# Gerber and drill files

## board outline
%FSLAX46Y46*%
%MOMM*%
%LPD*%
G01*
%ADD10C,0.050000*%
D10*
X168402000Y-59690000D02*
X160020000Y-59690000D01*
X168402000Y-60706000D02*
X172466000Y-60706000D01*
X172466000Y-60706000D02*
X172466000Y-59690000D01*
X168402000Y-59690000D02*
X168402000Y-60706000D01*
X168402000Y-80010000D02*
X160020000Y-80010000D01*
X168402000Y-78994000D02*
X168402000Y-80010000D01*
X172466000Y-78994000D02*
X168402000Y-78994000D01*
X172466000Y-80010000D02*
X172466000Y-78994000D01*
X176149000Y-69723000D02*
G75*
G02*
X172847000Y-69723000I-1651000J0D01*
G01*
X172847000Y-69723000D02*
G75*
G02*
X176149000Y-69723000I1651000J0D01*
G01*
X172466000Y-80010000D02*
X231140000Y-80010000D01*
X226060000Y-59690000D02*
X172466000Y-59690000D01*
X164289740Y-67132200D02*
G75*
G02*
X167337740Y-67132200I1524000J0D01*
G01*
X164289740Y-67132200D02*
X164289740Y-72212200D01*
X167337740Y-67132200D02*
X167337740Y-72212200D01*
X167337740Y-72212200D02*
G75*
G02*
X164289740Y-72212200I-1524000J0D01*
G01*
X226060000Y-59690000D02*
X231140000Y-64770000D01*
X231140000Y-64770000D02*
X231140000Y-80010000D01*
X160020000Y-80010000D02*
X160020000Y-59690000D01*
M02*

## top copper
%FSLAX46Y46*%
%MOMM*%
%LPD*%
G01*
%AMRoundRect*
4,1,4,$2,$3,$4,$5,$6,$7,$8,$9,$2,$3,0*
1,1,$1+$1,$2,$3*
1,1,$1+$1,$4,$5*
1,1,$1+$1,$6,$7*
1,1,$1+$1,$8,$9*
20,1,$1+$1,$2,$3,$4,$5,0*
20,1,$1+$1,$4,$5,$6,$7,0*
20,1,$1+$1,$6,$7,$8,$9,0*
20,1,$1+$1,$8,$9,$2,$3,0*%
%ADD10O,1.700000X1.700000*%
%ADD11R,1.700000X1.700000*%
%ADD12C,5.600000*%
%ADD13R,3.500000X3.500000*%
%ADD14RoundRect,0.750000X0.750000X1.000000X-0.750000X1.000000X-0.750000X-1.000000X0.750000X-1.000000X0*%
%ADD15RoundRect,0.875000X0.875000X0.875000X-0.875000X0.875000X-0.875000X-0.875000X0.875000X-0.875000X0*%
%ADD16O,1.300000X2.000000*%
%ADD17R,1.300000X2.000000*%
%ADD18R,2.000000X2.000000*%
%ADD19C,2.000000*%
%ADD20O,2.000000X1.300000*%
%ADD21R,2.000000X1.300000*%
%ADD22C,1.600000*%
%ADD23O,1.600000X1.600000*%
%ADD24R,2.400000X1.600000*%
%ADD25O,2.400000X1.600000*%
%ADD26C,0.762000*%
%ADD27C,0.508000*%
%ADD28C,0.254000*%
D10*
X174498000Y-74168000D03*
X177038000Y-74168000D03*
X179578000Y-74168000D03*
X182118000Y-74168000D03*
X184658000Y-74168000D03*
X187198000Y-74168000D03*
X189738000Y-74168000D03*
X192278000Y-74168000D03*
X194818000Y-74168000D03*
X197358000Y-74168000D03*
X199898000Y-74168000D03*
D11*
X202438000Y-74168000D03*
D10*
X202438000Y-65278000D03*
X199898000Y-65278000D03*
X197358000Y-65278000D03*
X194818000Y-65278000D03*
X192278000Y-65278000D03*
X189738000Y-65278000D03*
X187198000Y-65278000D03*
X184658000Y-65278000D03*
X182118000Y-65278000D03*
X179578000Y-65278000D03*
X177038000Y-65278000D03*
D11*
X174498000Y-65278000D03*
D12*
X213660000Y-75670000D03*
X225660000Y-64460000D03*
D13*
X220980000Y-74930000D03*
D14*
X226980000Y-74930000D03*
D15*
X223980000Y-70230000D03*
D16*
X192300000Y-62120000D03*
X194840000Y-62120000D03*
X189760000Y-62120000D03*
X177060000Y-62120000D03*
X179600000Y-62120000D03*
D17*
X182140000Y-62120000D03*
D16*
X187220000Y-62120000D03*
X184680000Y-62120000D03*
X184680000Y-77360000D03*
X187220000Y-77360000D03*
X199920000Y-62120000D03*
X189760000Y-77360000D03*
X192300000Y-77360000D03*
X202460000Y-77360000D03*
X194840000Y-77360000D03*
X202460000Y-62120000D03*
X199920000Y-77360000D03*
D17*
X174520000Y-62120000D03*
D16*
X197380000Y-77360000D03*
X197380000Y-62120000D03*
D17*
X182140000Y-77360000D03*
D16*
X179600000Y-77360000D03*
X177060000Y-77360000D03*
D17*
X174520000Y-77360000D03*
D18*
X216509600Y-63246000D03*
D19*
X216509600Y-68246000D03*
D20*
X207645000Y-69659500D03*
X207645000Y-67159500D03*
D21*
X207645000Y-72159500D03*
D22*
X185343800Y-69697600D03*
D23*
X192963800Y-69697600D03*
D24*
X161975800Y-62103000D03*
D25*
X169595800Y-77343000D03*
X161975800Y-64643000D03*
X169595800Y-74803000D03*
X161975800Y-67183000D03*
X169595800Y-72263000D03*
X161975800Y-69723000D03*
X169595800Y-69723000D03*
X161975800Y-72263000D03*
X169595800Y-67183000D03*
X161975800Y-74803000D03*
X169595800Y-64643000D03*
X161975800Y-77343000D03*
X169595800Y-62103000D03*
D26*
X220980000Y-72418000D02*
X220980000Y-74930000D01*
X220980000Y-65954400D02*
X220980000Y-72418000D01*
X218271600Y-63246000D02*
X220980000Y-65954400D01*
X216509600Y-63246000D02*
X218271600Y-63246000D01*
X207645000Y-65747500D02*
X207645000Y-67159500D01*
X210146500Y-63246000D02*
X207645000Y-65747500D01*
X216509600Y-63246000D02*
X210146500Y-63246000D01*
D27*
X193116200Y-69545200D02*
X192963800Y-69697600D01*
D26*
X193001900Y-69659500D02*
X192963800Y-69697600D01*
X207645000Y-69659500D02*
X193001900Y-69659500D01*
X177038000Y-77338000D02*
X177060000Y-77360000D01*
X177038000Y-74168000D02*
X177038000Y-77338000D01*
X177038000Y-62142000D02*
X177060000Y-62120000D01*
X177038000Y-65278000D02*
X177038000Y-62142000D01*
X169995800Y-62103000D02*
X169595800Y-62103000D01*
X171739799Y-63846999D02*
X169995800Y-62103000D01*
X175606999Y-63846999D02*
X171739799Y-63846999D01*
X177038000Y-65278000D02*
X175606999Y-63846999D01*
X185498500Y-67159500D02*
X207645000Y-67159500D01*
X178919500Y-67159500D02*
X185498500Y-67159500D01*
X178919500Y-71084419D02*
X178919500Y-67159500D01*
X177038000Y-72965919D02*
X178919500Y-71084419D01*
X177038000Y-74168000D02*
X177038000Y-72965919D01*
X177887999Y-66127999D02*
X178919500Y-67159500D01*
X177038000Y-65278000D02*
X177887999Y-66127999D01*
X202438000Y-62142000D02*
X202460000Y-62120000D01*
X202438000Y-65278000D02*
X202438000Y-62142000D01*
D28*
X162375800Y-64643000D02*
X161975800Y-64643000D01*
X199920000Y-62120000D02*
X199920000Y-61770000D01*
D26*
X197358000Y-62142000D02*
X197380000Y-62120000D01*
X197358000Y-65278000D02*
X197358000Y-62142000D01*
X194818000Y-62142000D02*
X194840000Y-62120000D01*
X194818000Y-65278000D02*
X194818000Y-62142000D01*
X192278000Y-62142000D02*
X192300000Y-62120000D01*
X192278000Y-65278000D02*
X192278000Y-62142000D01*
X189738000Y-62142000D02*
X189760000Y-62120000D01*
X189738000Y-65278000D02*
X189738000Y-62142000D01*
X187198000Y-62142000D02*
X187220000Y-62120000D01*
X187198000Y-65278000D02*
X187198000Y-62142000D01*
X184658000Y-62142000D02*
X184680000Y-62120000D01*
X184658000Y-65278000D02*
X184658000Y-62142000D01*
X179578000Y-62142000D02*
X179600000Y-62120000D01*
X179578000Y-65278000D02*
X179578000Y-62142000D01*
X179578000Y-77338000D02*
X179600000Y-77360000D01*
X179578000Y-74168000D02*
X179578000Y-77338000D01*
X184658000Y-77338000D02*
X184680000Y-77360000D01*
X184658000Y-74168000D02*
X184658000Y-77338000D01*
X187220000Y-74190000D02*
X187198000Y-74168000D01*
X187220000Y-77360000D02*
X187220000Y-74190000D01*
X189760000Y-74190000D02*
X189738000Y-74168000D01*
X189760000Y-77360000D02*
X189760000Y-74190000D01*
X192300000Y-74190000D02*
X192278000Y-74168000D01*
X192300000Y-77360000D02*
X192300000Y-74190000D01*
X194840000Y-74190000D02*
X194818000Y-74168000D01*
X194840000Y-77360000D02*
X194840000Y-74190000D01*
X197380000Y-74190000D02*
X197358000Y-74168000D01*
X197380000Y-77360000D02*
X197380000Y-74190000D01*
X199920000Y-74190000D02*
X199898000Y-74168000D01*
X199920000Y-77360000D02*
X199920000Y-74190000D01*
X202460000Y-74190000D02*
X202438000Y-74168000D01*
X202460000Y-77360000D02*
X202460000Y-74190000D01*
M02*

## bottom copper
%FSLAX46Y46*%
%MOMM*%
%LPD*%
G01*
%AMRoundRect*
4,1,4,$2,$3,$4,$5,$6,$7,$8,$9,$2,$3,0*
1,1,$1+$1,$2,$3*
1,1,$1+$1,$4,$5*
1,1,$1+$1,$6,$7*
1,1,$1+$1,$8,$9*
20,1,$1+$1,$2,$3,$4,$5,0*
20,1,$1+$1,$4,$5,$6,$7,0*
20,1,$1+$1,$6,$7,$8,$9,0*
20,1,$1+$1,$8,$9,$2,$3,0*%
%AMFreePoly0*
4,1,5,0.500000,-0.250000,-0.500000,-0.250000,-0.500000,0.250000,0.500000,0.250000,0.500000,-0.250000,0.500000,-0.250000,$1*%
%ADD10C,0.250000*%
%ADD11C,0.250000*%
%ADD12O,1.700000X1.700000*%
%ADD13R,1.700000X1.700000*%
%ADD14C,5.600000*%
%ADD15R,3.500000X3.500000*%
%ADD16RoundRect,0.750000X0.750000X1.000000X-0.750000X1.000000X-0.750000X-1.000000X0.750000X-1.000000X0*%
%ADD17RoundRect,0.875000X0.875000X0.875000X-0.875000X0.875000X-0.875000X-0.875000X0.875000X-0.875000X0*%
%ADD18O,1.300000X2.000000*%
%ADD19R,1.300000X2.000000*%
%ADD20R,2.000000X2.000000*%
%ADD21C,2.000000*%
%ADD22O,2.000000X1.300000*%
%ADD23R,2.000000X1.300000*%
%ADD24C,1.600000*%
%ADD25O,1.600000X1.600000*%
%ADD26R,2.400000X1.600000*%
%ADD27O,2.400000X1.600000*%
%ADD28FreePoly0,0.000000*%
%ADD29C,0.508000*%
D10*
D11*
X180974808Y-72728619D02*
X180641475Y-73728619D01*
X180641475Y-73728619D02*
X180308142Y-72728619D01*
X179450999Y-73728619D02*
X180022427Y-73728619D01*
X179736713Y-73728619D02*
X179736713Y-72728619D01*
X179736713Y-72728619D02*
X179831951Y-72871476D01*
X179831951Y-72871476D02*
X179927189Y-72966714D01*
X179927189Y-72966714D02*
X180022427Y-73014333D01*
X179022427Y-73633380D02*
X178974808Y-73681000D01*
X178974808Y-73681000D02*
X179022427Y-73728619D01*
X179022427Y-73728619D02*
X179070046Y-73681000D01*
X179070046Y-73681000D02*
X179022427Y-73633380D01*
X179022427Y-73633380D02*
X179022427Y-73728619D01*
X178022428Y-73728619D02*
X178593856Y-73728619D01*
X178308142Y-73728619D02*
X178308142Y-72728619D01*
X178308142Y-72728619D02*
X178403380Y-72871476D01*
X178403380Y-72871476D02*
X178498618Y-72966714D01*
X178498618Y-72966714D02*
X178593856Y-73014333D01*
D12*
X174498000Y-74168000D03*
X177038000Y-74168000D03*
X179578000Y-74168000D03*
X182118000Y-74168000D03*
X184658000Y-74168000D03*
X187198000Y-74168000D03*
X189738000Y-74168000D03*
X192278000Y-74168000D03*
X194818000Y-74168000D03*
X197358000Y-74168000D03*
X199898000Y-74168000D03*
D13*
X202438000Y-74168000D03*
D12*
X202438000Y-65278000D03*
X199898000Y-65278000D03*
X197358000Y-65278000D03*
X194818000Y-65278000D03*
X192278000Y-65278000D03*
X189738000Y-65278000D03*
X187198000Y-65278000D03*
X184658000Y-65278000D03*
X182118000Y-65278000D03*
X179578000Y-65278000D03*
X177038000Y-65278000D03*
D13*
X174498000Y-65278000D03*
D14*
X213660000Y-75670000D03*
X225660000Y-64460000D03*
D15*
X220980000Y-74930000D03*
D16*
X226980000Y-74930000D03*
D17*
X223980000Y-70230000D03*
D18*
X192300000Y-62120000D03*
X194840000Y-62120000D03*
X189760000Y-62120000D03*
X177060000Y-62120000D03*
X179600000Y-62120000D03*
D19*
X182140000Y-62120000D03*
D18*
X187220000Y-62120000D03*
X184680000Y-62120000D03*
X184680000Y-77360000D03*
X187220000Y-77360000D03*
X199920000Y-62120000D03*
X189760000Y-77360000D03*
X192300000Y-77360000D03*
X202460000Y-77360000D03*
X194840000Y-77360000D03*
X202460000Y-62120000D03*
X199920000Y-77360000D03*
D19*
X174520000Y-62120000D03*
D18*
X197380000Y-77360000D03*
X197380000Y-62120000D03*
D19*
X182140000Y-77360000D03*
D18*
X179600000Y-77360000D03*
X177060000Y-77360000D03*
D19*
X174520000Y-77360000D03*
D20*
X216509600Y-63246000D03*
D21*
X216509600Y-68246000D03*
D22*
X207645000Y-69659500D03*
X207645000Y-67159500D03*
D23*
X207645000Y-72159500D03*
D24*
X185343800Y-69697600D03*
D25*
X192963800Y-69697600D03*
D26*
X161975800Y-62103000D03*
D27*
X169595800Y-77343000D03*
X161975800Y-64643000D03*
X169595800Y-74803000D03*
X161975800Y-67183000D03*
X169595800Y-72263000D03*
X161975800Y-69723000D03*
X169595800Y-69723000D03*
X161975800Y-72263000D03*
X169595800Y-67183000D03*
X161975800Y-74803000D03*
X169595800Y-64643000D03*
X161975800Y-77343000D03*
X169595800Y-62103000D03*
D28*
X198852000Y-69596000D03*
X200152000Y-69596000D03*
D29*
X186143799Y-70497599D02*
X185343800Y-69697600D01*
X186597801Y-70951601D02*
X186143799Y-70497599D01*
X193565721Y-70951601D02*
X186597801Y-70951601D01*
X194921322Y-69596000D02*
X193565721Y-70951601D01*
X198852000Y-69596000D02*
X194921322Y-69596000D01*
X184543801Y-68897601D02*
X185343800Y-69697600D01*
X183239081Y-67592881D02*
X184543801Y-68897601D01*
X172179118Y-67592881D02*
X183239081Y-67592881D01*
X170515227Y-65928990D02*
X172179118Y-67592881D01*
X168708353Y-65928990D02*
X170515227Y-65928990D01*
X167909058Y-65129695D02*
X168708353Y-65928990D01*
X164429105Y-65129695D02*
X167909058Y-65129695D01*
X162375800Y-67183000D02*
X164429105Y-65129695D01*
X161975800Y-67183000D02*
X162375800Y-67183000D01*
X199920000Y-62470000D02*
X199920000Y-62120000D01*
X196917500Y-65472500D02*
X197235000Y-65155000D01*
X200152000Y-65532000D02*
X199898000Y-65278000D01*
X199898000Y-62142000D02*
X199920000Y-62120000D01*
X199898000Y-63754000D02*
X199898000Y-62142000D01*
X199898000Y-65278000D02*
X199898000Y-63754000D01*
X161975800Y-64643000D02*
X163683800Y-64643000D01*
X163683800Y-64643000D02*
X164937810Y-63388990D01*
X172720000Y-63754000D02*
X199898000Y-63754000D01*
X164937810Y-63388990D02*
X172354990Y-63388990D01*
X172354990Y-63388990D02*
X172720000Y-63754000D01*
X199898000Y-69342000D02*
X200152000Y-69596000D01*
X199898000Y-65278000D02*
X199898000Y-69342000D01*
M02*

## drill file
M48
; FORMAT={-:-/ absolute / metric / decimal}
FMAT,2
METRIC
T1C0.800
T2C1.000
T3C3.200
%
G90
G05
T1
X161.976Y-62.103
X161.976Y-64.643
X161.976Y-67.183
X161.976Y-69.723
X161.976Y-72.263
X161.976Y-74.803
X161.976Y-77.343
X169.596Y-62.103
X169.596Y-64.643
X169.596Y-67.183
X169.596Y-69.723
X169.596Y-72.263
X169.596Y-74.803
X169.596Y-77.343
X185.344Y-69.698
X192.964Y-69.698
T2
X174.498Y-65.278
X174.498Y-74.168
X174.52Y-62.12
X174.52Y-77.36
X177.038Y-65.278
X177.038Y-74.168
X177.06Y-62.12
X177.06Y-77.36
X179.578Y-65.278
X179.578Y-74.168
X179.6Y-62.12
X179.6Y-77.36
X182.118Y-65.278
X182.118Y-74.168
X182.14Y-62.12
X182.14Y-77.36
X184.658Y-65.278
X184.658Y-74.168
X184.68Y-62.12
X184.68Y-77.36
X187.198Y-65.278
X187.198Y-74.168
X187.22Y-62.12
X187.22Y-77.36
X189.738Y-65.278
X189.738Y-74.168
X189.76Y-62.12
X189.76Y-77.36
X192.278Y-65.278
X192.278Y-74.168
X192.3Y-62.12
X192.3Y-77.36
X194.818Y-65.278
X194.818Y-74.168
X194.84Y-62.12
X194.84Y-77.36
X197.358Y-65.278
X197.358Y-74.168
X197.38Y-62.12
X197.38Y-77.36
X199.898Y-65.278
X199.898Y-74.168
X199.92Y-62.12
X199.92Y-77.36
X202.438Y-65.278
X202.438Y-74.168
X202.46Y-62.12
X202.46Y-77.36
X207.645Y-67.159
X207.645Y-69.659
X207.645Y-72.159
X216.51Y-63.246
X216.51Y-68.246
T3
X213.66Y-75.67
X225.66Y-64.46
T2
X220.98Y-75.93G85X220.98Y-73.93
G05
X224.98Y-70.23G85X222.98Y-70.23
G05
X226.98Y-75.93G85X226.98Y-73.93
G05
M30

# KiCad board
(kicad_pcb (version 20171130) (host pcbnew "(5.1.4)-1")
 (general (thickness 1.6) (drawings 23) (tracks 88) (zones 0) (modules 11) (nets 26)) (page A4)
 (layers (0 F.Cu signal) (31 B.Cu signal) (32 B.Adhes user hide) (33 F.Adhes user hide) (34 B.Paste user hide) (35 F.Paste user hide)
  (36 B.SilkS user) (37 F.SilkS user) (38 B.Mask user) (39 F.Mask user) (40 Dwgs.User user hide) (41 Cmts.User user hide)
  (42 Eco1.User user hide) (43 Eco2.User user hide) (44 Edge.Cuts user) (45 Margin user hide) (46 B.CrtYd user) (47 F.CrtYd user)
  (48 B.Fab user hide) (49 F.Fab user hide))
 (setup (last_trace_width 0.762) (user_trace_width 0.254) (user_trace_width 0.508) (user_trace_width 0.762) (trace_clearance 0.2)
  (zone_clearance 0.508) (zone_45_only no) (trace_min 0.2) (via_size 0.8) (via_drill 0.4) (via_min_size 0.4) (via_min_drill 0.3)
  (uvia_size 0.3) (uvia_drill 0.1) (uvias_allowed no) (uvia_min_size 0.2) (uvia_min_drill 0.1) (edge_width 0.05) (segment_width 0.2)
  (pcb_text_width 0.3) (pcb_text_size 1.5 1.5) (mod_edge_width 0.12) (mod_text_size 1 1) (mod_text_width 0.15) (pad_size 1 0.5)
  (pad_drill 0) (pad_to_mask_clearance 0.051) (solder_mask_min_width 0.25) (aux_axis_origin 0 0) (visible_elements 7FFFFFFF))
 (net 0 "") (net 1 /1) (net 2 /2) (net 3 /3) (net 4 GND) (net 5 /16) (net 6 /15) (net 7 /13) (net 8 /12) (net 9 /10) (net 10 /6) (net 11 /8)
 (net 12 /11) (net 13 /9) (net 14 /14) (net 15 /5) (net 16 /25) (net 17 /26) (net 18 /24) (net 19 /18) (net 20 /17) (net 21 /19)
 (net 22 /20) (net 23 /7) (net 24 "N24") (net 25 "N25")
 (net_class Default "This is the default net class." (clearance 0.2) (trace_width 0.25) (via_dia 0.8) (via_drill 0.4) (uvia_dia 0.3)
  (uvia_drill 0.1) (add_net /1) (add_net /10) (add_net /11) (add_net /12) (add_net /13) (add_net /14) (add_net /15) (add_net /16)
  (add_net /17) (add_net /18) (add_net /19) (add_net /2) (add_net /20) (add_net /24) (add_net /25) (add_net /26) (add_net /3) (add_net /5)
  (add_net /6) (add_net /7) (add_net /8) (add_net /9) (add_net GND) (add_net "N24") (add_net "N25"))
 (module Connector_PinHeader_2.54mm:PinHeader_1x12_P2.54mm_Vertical (layer F.Cu) (at 202.438 74.168 270)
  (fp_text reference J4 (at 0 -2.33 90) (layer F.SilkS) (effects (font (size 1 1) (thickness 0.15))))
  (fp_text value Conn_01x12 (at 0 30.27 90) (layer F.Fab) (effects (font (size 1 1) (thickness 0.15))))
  (pad 12 thru_hole oval (at 0 27.94 270) (size 1.7 1.7) (drill 1) (layers *.Cu *.Mask) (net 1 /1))
  (pad 11 thru_hole oval (at 0 25.4 270) (size 1.7 1.7) (drill 1) (layers *.Cu *.Mask) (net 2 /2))
  (pad 10 thru_hole oval (at 0 22.86 270) (size 1.7 1.7) (drill 1) (layers *.Cu *.Mask) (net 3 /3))
  (pad 9 thru_hole oval (at 0 20.32 270) (size 1.7 1.7) (drill 1) (layers *.Cu *.Mask) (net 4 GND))
  (pad 8 thru_hole oval (at 0 17.78 270) (size 1.7 1.7) (drill 1) (layers *.Cu *.Mask) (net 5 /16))
  (pad 7 thru_hole oval (at 0 15.24 270) (size 1.7 1.7) (drill 1) (layers *.Cu *.Mask) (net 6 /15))
  (pad 6 thru_hole oval (at 0 12.7 270) (size 1.7 1.7) (drill 1) (layers *.Cu *.Mask) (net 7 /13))
  (pad 5 thru_hole oval (at 0 10.16 270) (size 1.7 1.7) (drill 1) (layers *.Cu *.Mask) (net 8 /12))
  (pad 4 thru_hole oval (at 0 7.62 270) (size 1.7 1.7) (drill 1) (layers *.Cu *.Mask) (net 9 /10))
  (pad 3 thru_hole oval (at 0 5.08 270) (size 1.7 1.7) (drill 1) (layers *.Cu *.Mask) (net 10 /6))
  (pad 2 thru_hole oval (at 0 2.54 270) (size 1.7 1.7) (drill 1) (layers *.Cu *.Mask) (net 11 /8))
  (pad 1 thru_hole rect (at 0 0 270) (size 1.7 1.7) (drill 1) (layers *.Cu *.Mask) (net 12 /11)))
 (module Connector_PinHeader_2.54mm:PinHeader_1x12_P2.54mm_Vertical (layer F.Cu) (at 174.498 65.278 90)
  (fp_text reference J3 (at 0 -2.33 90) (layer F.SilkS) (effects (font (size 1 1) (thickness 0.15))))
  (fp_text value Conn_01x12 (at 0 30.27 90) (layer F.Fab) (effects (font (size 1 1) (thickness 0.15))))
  (pad 12 thru_hole oval (at 0 27.94 90) (size 1.7 1.7) (drill 1) (layers *.Cu *.Mask) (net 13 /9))
  (pad 11 thru_hole oval (at 0 25.4 90) (size 1.7 1.7) (drill 1) (layers *.Cu *.Mask) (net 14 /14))
  (pad 10 thru_hole oval (at 0 22.86 90) (size 1.7 1.7) (drill 1) (layers *.Cu *.Mask) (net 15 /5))
  (pad 9 thru_hole oval (at 0 20.32 90) (size 1.7 1.7) (drill 1) (layers *.Cu *.Mask) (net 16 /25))
  (pad 8 thru_hole oval (at 0 17.78 90) (size 1.7 1.7) (drill 1) (layers *.Cu *.Mask) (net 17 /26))
  (pad 7 thru_hole oval (at 0 15.24 90) (size 1.7 1.7) (drill 1) (layers *.Cu *.Mask) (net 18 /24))
  (pad 6 thru_hole oval (at 0 12.7 90) (size 1.7 1.7) (drill 1) (layers *.Cu *.Mask) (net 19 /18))
  (pad 5 thru_hole oval (at 0 10.16 90) (size 1.7 1.7) (drill 1) (layers *.Cu *.Mask) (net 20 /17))
  (pad 4 thru_hole oval (at 0 7.62 90) (size 1.7 1.7) (drill 1) (layers *.Cu *.Mask) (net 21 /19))
  (pad 3 thru_hole oval (at 0 5.08 90) (size 1.7 1.7) (drill 1) (layers *.Cu *.Mask) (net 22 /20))
  (pad 2 thru_hole oval (at 0 2.54 90) (size 1.7 1.7) (drill 1) (layers *.Cu *.Mask) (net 2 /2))
  (pad 1 thru_hole rect (at 0 0 90) (size 1.7 1.7) (drill 1) (layers *.Cu *.Mask) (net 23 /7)))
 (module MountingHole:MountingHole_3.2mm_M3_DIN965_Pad (layer F.Cu) (at 213.66 75.67)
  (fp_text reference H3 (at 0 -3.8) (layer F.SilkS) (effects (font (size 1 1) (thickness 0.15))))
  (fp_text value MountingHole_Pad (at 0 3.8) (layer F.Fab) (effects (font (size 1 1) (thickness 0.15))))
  (pad 1 thru_hole circle (at 0 0) (size 5.6 5.6) (drill 3.2) (layers *.Cu *.Mask) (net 4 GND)))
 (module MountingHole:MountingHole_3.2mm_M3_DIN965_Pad (layer F.Cu) (at 225.66 64.46)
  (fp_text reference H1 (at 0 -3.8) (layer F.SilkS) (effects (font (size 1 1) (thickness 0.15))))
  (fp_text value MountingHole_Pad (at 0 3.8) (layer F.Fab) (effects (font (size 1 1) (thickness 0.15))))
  (pad 1 thru_hole circle (at 0 0) (size 5.6 5.6) (drill 3.2) (layers *.Cu *.Mask) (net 4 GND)))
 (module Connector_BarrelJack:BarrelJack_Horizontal (layer F.Cu) (at 220.98 74.93 180)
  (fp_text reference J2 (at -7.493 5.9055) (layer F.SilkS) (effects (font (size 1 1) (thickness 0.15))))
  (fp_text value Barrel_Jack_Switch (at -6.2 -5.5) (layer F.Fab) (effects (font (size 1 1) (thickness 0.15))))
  (pad 1 thru_hole rect (at 0 0 180) (size 3.5 3.5) (drill oval 1 3) (layers *.Cu *.Mask) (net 2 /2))
  (pad 2 thru_hole roundrect (at -6 0 180) (size 3 3.5) (drill oval 1 3) (layers *.Cu *.Mask) (roundrect_rratio 0.25) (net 1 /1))
  (pad 3 thru_hole roundrect (at -3 4.7 180) (size 3.5 3.5) (drill oval 3 1) (layers *.Cu *.Mask) (roundrect_rratio 0.25) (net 1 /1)))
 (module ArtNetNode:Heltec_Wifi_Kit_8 (layer F.Cu) (at 160.02 78.74)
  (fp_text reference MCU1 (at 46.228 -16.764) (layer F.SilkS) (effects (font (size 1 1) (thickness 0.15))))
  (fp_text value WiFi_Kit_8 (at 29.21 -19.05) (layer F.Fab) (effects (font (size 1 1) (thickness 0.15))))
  (pad 26 thru_hole oval (at 32.28 -16.62) (size 1.3 2) (drill 1) (layers *.Cu *.Mask) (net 17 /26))
  (pad 25 thru_hole oval (at 34.82 -16.62) (size 1.3 2) (drill 1) (layers *.Cu *.Mask) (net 16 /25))
  (pad 24 thru_hole oval (at 29.74 -16.62) (size 1.3 2) (drill 1) (layers *.Cu *.Mask) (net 18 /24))
  (pad 21 thru_hole oval (at 17.04 -16.62) (size 1.3 2) (drill 1) (layers *.Cu *.Mask) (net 2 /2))
  (pad 20 thru_hole oval (at 19.58 -16.62) (size 1.3 2) (drill 1) (layers *.Cu *.Mask) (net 22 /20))
  (pad 19 thru_hole rect (at 22.12 -16.62) (size 1.3 2) (drill 1) (layers *.Cu *.Mask) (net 21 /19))
  (pad 18 thru_hole oval (at 27.2 -16.62) (size 1.3 2) (drill 1) (layers *.Cu *.Mask) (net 19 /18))
  (pad 17 thru_hole oval (at 24.66 -16.62) (size 1.3 2) (drill 1) (layers *.Cu *.Mask) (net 20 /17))
  (pad 16 thru_hole oval (at 24.66 -1.38) (size 1.3 2) (drill 1) (layers *.Cu *.Mask) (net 5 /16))
  (pad 15 thru_hole oval (at 27.2 -1.38) (size 1.3 2) (drill 1) (layers *.Cu *.Mask) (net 6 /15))
  (pad 14 thru_hole oval (at 39.9 -16.62) (size 1.3 2) (drill 1) (layers *.Cu *.Mask) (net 14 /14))
  (pad 13 thru_hole oval (at 29.74 -1.38) (size 1.3 2) (drill 1) (layers *.Cu *.Mask) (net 7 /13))
  (pad 12 thru_hole oval (at 32.28 -1.38) (size 1.3 2) (drill 1) (layers *.Cu *.Mask) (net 8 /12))
  (pad 11 thru_hole oval (at 42.44 -1.38) (size 1.3 2) (drill 1) (layers *.Cu *.Mask) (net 12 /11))
  (pad 10 thru_hole oval (at 34.82 -1.38) (size 1.3 2) (drill 1) (layers *.Cu *.Mask) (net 9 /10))
  (pad 9 thru_hole oval (at 42.44 -16.62) (size 1.3 2) (drill 1) (layers *.Cu *.Mask) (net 13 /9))
  (pad 8 thru_hole oval (at 39.9 -1.38) (size 1.3 2) (drill 1) (layers *.Cu *.Mask) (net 11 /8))
  (pad 7 thru_hole rect (at 14.5 -16.62) (size 1.3 2) (drill 1) (layers *.Cu *.Mask) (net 23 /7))
  (pad 6 thru_hole oval (at 37.36 -1.38) (size 1.3 2) (drill 1) (layers *.Cu *.Mask) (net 10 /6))
  (pad 5 thru_hole oval (at 37.36 -16.62) (size 1.3 2) (drill 1) (layers *.Cu *.Mask) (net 15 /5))
  (pad 4 thru_hole rect (at 22.12 -1.38) (size 1.3 2) (drill 1) (layers *.Cu *.Mask) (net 4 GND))
  (pad 3 thru_hole oval (at 19.58 -1.38) (size 1.3 2) (drill 1) (layers *.Cu *.Mask) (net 3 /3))
  (pad 2 thru_hole oval (at 17.04 -1.38) (size 1.3 2) (drill 1) (layers *.Cu *.Mask) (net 2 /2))
  (pad 1 thru_hole rect (at 14.5 -1.38) (size 1.3 2) (drill 1) (layers *.Cu *.Mask) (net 1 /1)))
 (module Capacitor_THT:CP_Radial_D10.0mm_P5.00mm (layer F.Cu) (at 216.5096 63.246 270)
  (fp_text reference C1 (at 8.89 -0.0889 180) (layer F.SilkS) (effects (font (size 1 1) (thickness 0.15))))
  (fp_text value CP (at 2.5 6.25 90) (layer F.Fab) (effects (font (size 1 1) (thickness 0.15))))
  (pad 1 thru_hole rect (at 0 0 270) (size 2 2) (drill 1) (layers *.Cu *.Mask) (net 2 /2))
  (pad 2 thru_hole circle (at 5 0 270) (size 2 2) (drill 1) (layers *.Cu *.Mask) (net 1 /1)))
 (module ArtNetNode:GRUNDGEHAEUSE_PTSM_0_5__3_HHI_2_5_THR (layer F.Cu) (at 204.645 69.6595)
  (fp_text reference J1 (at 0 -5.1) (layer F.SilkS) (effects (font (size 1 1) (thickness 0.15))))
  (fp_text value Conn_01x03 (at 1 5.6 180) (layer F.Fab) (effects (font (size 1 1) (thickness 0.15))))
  (pad 2 thru_hole oval (at 3 0 270) (size 1.3 2) (drill 1) (layers *.Cu *.Mask) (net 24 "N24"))
  (pad 1 thru_hole oval (at 3 -2.5 270) (size 1.3 2) (drill 1) (layers *.Cu *.Mask) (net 2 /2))
  (pad 3 thru_hole rect (at 3 2.5 270) (size 1.3 2) (drill 1) (layers *.Cu *.Mask) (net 1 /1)))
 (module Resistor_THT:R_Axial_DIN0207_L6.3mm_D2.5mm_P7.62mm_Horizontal (layer F.Cu) (at 185.3438 69.6976)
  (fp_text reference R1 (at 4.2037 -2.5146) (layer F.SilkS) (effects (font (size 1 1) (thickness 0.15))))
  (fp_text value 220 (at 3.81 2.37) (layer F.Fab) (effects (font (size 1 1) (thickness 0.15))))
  (pad 1 thru_hole circle (at 0 0) (size 1.6 1.6) (drill 0.8) (layers *.Cu *.Mask) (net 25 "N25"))
  (pad 2 thru_hole oval (at 7.62 0) (size 1.6 1.6) (drill 0.8) (layers *.Cu *.Mask) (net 24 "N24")))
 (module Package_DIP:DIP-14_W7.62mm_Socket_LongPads (layer F.Cu) (at 161.9758 62.103)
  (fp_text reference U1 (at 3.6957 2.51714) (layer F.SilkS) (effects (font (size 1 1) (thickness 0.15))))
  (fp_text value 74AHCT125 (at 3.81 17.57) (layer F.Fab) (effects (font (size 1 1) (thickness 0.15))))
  (pad 1 thru_hole rect (at 0 0) (size 2.4 1.6) (drill 0.8) (layers *.Cu *.Mask) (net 1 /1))
  (pad 8 thru_hole oval (at 7.62 15.24) (size 2.4 1.6) (drill 0.8) (layers *.Cu *.Mask))
  (pad 2 thru_hole oval (at 0 2.54) (size 2.4 1.6) (drill 0.8) (layers *.Cu *.Mask) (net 14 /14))
  (pad 9 thru_hole oval (at 7.62 12.7) (size 2.4 1.6) (drill 0.8) (layers *.Cu *.Mask))
  (pad 3 thru_hole oval (at 0 5.08) (size 2.4 1.6) (drill 0.8) (layers *.Cu *.Mask) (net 25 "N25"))
  (pad 10 thru_hole oval (at 7.62 10.16) (size 2.4 1.6) (drill 0.8) (layers *.Cu *.Mask))
  (pad 4 thru_hole oval (at 0 7.62) (size 2.4 1.6) (drill 0.8) (layers *.Cu *.Mask))
  (pad 11 thru_hole oval (at 7.62 7.62) (size 2.4 1.6) (drill 0.8) (layers *.Cu *.Mask))
  (pad 5 thru_hole oval (at 0 10.16) (size 2.4 1.6) (drill 0.8) (layers *.Cu *.Mask))
  (pad 12 thru_hole oval (at 7.62 5.08) (size 2.4 1.6) (drill 0.8) (layers *.Cu *.Mask))
  (pad 6 thru_hole oval (at 0 12.7) (size 2.4 1.6) (drill 0.8) (layers *.Cu *.Mask))
  (pad 13 thru_hole oval (at 7.62 2.54) (size 2.4 1.6) (drill 0.8) (layers *.Cu *.Mask))
  (pad 7 thru_hole oval (at 0 15.24) (size 2.4 1.6) (drill 0.8) (layers *.Cu *.Mask) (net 1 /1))
  (pad 14 thru_hole oval (at 7.62 0) (size 2.4 1.6) (drill 0.8) (layers *.Cu *.Mask) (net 2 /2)))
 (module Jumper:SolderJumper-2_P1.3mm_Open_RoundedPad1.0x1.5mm (layer B.Cu) (at 199.502 69.596)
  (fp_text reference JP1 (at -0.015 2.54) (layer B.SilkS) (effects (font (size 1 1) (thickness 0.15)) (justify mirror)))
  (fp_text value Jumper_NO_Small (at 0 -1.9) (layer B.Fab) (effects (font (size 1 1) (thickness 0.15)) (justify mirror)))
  (pad 1 smd custom (at -0.65 0) (size 1 0.5) (layers B.Cu B.Mask) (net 25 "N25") (zone_connect 2)
   (options (clearance outline) (anchor rect)) (primitives))
  (pad 2 smd custom (at 0.65 0) (size 1 0.5) (layers B.Cu B.Mask) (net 14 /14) (zone_connect 2) (options (clearance outline) (anchor rect))
   (primitives)))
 (gr_line (start 168.402 59.69) (end 160.02 59.69) (layer Edge.Cuts) (width 0.05))
 (gr_line (start 168.402 60.706) (end 172.466 60.706) (layer Edge.Cuts) (width 0.05))
 (gr_line (start 172.466 60.706) (end 172.466 59.69) (layer Edge.Cuts) (width 0.05))
 (gr_line (start 168.402 59.69) (end 168.402 60.706) (layer Edge.Cuts) (width 0.05))
 (gr_line (start 168.402 80.01) (end 160.02 80.01) (layer Edge.Cuts) (width 0.05))
 (gr_line (start 168.402 78.994) (end 168.402 80.01) (layer Edge.Cuts) (width 0.05))
 (gr_line (start 172.466 78.994) (end 168.402 78.994) (layer Edge.Cuts) (width 0.05))
 (gr_line (start 172.466 80.01) (end 172.466 78.994) (layer Edge.Cuts) (width 0.05))
 (gr_circle (center 174.498 69.723) (end 176.149 69.723) (layer Edge.Cuts) (width 0.05))
 (gr_line (start 172.466 80.01) (end 231.14 80.01) (layer Edge.Cuts) (width 0.05))
 (gr_line (start 226.06 59.69) (end 172.466 59.69) (layer Edge.Cuts) (width 0.05))
 (gr_arc (start 165.81374 67.1322) (end 167.33774 67.1322) (angle -180) (layer Edge.Cuts) (width 0.05))
 (gr_line (start 164.28974 67.1322) (end 164.28974 72.2122) (layer Edge.Cuts) (width 0.05))
 (gr_line (start 167.33774 67.1322) (end 167.33774 72.2122) (layer Edge.Cuts) (width 0.05))
 (gr_arc (start 165.81374 72.2122) (end 164.28974 72.2122) (angle -180) (layer Edge.Cuts) (width 0.05))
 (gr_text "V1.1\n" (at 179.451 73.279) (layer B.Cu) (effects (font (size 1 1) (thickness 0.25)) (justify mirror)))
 (gr_line (start 226.06 59.69) (end 231.14 64.77) (layer Edge.Cuts) (width 0.05))
 (gr_line (start 231.14 64.77) (end 231.14 80.01) (layer Edge.Cuts) (width 0.05))
 (gr_line (start 160.02 80.01) (end 160.02 59.69) (layer Edge.Cuts) (width 0.05))
 (segment (start 220.98 72.418) (end 220.98 74.93) (width 0.762) (layer F.Cu) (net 2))
 (segment (start 220.98 65.9544) (end 220.98 72.418) (width 0.762) (layer F.Cu) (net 2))
 (segment (start 218.2716 63.246) (end 220.98 65.9544) (width 0.762) (layer F.Cu) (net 2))
 (segment (start 216.5096 63.246) (end 218.2716 63.246) (width 0.762) (layer F.Cu) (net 2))
 (segment (start 207.645 65.7475) (end 207.645 67.1595) (width 0.762) (layer F.Cu) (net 2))
 (segment (start 210.1465 63.246) (end 207.645 65.7475) (width 0.762) (layer F.Cu) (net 2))
 (segment (start 216.5096 63.246) (end 210.1465 63.246) (width 0.762) (layer F.Cu) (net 2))
 (segment (start 193.1162 69.5452) (end 192.9638 69.6976) (width 0.508) (layer F.Cu) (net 24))
 (segment (start 193.0019 69.6595) (end 192.9638 69.6976) (width 0.762) (layer F.Cu) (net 24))
 (segment (start 207.645 69.6595) (end 193.0019 69.6595) (width 0.762) (layer F.Cu) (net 24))
 (segment (start 186.143799 70.497599) (end 185.3438 69.6976) (width 0.508) (layer B.Cu) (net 25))
 (segment (start 186.597801 70.951601) (end 186.143799 70.497599) (width 0.508) (layer B.Cu) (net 25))
 (segment (start 193.565721 70.951601) (end 186.597801 70.951601) (width 0.508) (layer B.Cu) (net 25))
 (segment (start 194.921322 69.596) (end 193.565721 70.951601) (width 0.508) (layer B.Cu) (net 25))
 (segment (start 198.852 69.596) (end 194.921322 69.596) (width 0.508) (layer B.Cu) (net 25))
 (segment (start 184.543801 68.897601) (end 185.3438 69.6976) (width 0.508) (layer B.Cu) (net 25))
 (segment (start 183.239081 67.592881) (end 184.543801 68.897601) (width 0.508) (layer B.Cu) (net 25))
 (segment (start 172.179118 67.592881) (end 183.239081 67.592881) (width 0.508) (layer B.Cu) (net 25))
 (segment (start 170.515227 65.92899) (end 172.179118 67.592881) (width 0.508) (layer B.Cu) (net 25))
 (segment (start 168.708353 65.92899) (end 170.515227 65.92899) (width 0.508) (layer B.Cu) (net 25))
 (segment (start 167.909058 65.129695) (end 168.708353 65.92899) (width 0.508) (layer B.Cu) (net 25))
 (segment (start 164.429105 65.129695) (end 167.909058 65.129695) (width 0.508) (layer B.Cu) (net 25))
 (segment (start 162.3758 67.183) (end 164.429105 65.129695) (width 0.508) (layer B.Cu) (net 25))
 (segment (start 161.9758 67.183) (end 162.3758 67.183) (width 0.508) (layer B.Cu) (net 25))
 (segment (start 177.038 77.338) (end 177.06 77.36) (width 0.762) (layer F.Cu) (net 2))
 (segment (start 177.038 74.168) (end 177.038 77.338) (width 0.762) (layer F.Cu) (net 2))
 (segment (start 177.038 62.142) (end 177.06 62.12) (width 0.762) (layer F.Cu) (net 2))
 (segment (start 177.038 65.278) (end 177.038 62.142) (width 0.762) (layer F.Cu) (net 2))
 (segment (start 169.9958 62.103) (end 169.5958 62.103) (width 0.762) (layer F.Cu) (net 2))
 (segment (start 171.739799 63.846999) (end 169.9958 62.103) (width 0.762) (layer F.Cu) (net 2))
 (segment (start 175.606999 63.846999) (end 171.739799 63.846999) (width 0.762) (layer F.Cu) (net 2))
 (segment (start 177.038 65.278) (end 175.606999 63.846999) (width 0.762) (layer F.Cu) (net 2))
 (segment (start 185.4985 67.1595) (end 207.645 67.1595) (width 0.762) (layer F.Cu) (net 2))
 (segment (start 178.9195 67.1595) (end 185.4985 67.1595) (width 0.762) (layer F.Cu) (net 2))
 (segment (start 178.9195 71.084419) (end 178.9195 67.1595) (width 0.762) (layer F.Cu) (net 2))
 (segment (start 177.038 72.965919) (end 178.9195 71.084419) (width 0.762) (layer F.Cu) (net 2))
 (segment (start 177.038 74.168) (end 177.038 72.965919) (width 0.762) (layer F.Cu) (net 2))
 (segment (start 177.887999 66.127999) (end 178.9195 67.1595) (width 0.762) (layer F.Cu) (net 2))
 (segment (start 177.038 65.278) (end 177.887999 66.127999) (width 0.762) (layer F.Cu) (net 2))
 (segment (start 202.438 62.142) (end 202.46 62.12) (width 0.762) (layer F.Cu) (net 13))
 (segment (start 202.438 65.278) (end 202.438 62.142) (width 0.762) (layer F.Cu) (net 13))
 (segment (start 162.3758 64.643) (end 161.9758 64.643) (width 0.254) (layer F.Cu) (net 14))
 (segment (start 199.92 62.12) (end 199.92 61.77) (width 0.254) (layer F.Cu) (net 14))
 (segment (start 199.92 62.47) (end 199.92 62.12) (width 0.508) (layer B.Cu) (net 14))
 (segment (start 196.9175 65.4725) (end 197.235 65.155) (width 0.508) (layer B.Cu) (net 15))
 (segment (start 200.152 65.532) (end 199.898 65.278) (width 0.508) (layer B.Cu) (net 14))
 (segment (start 199.898 62.142) (end 199.92 62.12) (width 0.508) (layer B.Cu) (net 14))
 (segment (start 199.898 63.754) (end 199.898 62.142) (width 0.508) (layer B.Cu) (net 14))
 (segment (start 199.898 65.278) (end 199.898 63.754) (width 0.508) (layer B.Cu) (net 14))
 (segment (start 161.9758 64.643) (end 163.6838 64.643) (width 0.508) (layer B.Cu) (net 14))
 (segment (start 163.6838 64.643) (end 164.93781 63.38899) (width 0.508) (layer B.Cu) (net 14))
 (segment (start 172.72 63.754) (end 199.898 63.754) (width 0.508) (layer B.Cu) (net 14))
 (segment (start 164.93781 63.38899) (end 172.35499 63.38899) (width 0.508) (layer B.Cu) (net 14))
 (segment (start 172.35499 63.38899) (end 172.72 63.754) (width 0.508) (layer B.Cu) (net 14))
 (segment (start 199.898 69.342) (end 200.152 69.596) (width 0.508) (layer B.Cu) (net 14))
 (segment (start 199.898 65.278) (end 199.898 69.342) (width 0.508) (layer B.Cu) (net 14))
 (segment (start 197.358 62.142) (end 197.38 62.12) (width 0.762) (layer F.Cu) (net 15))
 (segment (start 197.358 65.278) (end 197.358 62.142) (width 0.762) (layer F.Cu) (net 15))
 (segment (start 194.818 62.142) (end 194.84 62.12) (width 0.762) (layer F.Cu) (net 16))
 (segment (start 194.818 65.278) (end 194.818 62.142) (width 0.762) (layer F.Cu) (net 16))
 (segment (start 192.278 62.142) (end 192.3 62.12) (width 0.762) (layer F.Cu) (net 17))
 (segment (start 192.278 65.278) (end 192.278 62.142) (width 0.762) (layer F.Cu) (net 17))
 (segment (start 189.738 62.142) (end 189.76 62.12) (width 0.762) (layer F.Cu) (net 18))
 (segment (start 189.738 65.278) (end 189.738 62.142) (width 0.762) (layer F.Cu) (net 18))
 (segment (start 187.198 62.142) (end 187.22 62.12) (width 0.762) (layer F.Cu) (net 19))
 (segment (start 187.198 65.278) (end 187.198 62.142) (width 0.762) (layer F.Cu) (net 19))
 (segment (start 184.658 62.142) (end 184.68 62.12) (width 0.762) (layer F.Cu) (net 20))
 (segment (start 184.658 65.278) (end 184.658 62.142) (width 0.762) (layer F.Cu) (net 20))
 (segment (start 179.578 62.142) (end 179.6 62.12) (width 0.762) (layer F.Cu) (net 22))
 (segment (start 179.578 65.278) (end 179.578 62.142) (width 0.762) (layer F.Cu) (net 22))
 (segment (start 179.578 77.338) (end 179.6 77.36) (width 0.762) (layer F.Cu) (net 3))
 (segment (start 179.578 74.168) (end 179.578 77.338) (width 0.762) (layer F.Cu) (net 3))
 (segment (start 184.658 77.338) (end 184.68 77.36) (width 0.762) (layer F.Cu) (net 5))
 (segment (start 184.658 74.168) (end 184.658 77.338) (width 0.762) (layer F.Cu) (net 5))
 (segment (start 187.22 74.19) (end 187.198 74.168) (width 0.762) (layer F.Cu) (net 6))
 (segment (start 187.22 77.36) (end 187.22 74.19) (width 0.762) (layer F.Cu) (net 6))
 (segment (start 189.76 74.19) (end 189.738 74.168) (width 0.762) (layer F.Cu) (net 7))
 (segment (start 189.76 77.36) (end 189.76 74.19) (width 0.762) (layer F.Cu) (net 7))
 (segment (start 192.3 74.19) (end 192.278 74.168) (width 0.762) (layer F.Cu) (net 8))
 (segment (start 192.3 77.36) (end 192.3 74.19) (width 0.762) (layer F.Cu) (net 8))
 (segment (start 194.84 74.19) (end 194.818 74.168) (width 0.762) (layer F.Cu) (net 9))
 (segment (start 194.84 77.36) (end 194.84 74.19) (width 0.762) (layer F.Cu) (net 9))
 (segment (start 197.38 74.19) (end 197.358 74.168) (width 0.762) (layer F.Cu) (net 10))
 (segment (start 197.38 77.36) (end 197.38 74.19) (width 0.762) (layer F.Cu) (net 10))
 (segment (start 199.92 74.19) (end 199.898 74.168) (width 0.762) (layer F.Cu) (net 11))
 (segment (start 199.92 77.36) (end 199.92 74.19) (width 0.762) (layer F.Cu) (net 11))
 (segment (start 202.46 74.19) (end 202.438 74.168) (width 0.762) (layer F.Cu) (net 12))
 (segment (start 202.46 77.36) (end 202.46 74.19) (width 0.762) (layer F.Cu) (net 12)))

